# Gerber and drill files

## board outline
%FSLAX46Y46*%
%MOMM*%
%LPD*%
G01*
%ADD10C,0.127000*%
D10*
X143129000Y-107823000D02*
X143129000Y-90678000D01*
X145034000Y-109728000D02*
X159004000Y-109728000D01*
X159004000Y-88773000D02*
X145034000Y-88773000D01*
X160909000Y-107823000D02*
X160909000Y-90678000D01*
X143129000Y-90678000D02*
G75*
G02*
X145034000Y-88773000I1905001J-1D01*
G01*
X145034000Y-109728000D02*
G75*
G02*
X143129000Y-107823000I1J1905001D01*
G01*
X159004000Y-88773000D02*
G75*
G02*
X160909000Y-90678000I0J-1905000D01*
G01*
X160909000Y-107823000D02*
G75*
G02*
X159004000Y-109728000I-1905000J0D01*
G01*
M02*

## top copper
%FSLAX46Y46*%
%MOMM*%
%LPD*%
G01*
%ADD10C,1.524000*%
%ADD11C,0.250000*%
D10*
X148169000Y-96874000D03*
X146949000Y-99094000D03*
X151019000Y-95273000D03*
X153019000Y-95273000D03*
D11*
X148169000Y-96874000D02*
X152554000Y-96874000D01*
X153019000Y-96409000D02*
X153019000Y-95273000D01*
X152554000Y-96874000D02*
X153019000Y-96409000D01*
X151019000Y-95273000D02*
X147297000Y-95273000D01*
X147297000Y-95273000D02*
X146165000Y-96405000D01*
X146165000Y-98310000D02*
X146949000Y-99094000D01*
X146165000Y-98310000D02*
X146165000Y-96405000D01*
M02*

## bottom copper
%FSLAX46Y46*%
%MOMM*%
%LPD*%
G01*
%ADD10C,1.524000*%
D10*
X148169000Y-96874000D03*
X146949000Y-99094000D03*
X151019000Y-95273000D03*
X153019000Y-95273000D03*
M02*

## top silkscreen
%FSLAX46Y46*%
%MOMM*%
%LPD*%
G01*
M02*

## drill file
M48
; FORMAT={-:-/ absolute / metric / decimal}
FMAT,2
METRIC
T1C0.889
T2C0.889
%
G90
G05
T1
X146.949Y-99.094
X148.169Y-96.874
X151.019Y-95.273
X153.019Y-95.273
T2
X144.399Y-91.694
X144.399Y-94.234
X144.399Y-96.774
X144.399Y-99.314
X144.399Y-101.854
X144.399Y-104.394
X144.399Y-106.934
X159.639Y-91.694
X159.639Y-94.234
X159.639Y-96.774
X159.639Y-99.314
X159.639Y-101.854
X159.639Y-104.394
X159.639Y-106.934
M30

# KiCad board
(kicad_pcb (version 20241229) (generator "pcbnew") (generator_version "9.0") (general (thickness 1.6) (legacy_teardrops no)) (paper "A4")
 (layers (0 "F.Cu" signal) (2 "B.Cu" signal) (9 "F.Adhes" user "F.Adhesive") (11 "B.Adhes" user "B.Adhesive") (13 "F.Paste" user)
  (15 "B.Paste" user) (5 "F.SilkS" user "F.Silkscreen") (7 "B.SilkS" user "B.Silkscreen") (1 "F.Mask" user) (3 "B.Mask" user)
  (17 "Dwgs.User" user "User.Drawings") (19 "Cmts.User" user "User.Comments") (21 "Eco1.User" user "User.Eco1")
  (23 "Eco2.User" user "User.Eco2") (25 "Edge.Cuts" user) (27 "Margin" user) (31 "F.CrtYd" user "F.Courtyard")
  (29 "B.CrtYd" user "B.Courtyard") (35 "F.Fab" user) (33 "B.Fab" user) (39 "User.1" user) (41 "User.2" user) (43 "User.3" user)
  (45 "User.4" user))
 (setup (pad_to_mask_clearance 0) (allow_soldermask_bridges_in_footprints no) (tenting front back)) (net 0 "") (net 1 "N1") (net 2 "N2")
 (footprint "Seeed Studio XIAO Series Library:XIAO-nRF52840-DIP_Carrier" (layer "F.Cu") (at 152.019 99.314)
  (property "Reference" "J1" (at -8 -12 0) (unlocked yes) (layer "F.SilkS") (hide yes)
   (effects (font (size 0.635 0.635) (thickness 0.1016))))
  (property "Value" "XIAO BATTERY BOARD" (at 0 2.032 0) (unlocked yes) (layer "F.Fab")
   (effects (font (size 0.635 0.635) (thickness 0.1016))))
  (fp_line (start -8.89 8.509) (end -8.89 -8.636) (stroke (width 0.127) (type solid)) (layer "Edge.Cuts"))
  (fp_line (start -6.985 10.414) (end 6.985 10.414) (stroke (width 0.127) (type solid)) (layer "Edge.Cuts"))
  (fp_line (start 6.985 -10.541) (end -6.985 -10.541) (stroke (width 0.127) (type solid)) (layer "Edge.Cuts"))
  (fp_line (start 8.89 8.509) (end 8.89 -8.636) (stroke (width 0.127) (type solid)) (layer "Edge.Cuts"))
  (fp_arc (start -8.89 -8.636) (mid -8.332038 -9.983038) (end -6.985 -10.541) (stroke (width 0.127) (type solid)) (layer "Edge.Cuts"))
  (fp_arc (start -6.985 10.414) (mid -8.332038 9.856038) (end -8.89 8.509) (stroke (width 0.127) (type solid)) (layer "Edge.Cuts"))
  (fp_arc (start 6.985 -10.541) (mid 8.332038 -9.983038) (end 8.89 -8.636) (stroke (width 0.127) (type solid)) (layer "Edge.Cuts"))
  (fp_arc (start 8.89 8.509) (mid 8.332038 9.856038) (end 6.985 10.414) (stroke (width 0.127) (type solid)) (layer "Edge.Cuts"))
  (pad "" np_thru_hole circle (at -7.62 -7.62 180) (size 1.524 1.524) (drill 0.889) (layers))
  (pad "" np_thru_hole circle (at -7.62 -5.08 180) (size 0.889 0.889) (drill 0.889) (layers))
  (pad "" np_thru_hole circle (at -7.62 -2.54 180) (size 1.524 1.524) (drill 0.889) (layers))
  (pad "" np_thru_hole circle (at -7.62 0 180) (size 1.524 1.524) (drill 0.889) (layers))
  (pad "" np_thru_hole circle (at -7.62 2.54 180) (size 1.524 1.524) (drill 0.889) (layers))
  (pad "" np_thru_hole circle (at -7.62 5.08 180) (size 1.524 1.524) (drill 0.889) (layers))
  (pad "" np_thru_hole circle (at -7.62 7.62 180) (size 1.524 1.524) (drill 0.889) (layers))
  (pad "" np_thru_hole circle (at 7.62 -7.62) (size 1.524 1.524) (drill 0.889) (layers))
  (pad "" np_thru_hole circle (at 7.62 -5.08) (size 1.524 1.524) (drill 0.889) (layers))
  (pad "" np_thru_hole circle (at 7.62 -2.54) (size 1.524 1.524) (drill 0.889) (layers))
  (pad "" np_thru_hole circle (at 7.62 0) (size 1.524 1.524) (drill 0.889) (layers))
  (pad "" np_thru_hole circle (at 7.62 2.54) (size 1.524 1.524) (drill 0.889) (layers))
  (pad "" np_thru_hole circle (at 7.62 5.08) (size 1.524 1.524) (drill 0.889) (layers))
  (pad "" np_thru_hole circle (at 7.62 7.62) (size 1.524 1.524) (drill 0.889) (layers))
  (pad "1" thru_hole circle (at -3.85 -2.44) (size 1.524 1.524) (drill 0.889) (layers "*.Cu" "*.Mask") (remove_unused_layers no)
   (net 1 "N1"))
  (pad "2" thru_hole circle (at -5.07 -0.22) (size 1.524 1.524) (drill 0.889) (layers "*.Cu" "*.Mask") (remove_unused_layers no)
   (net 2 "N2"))
  (pad "3" thru_hole circle (at -1 -4.041) (size 1.524 1.524) (drill 0.889) (layers "*.Cu" "*.Mask") (remove_unused_layers no) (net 2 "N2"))
  (pad "4" thru_hole circle (at 1 -4.041) (size 1.524 1.524) (drill 0.889) (layers "*.Cu" "*.Mask") (remove_unused_layers no) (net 1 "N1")))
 (segment (start 148.169 96.874) (end 152.554 96.874) (width 0.25) (layer "F.Cu") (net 1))
 (segment (start 153.019 96.409) (end 153.019 95.273) (width 0.25) (layer "F.Cu") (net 1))
 (segment (start 152.554 96.874) (end 153.019 96.409) (width 0.25) (layer "F.Cu") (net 1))
 (segment (start 151.019 95.273) (end 147.297 95.273) (width 0.25) (layer "F.Cu") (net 2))
 (segment (start 147.297 95.273) (end 146.165 96.405) (width 0.25) (layer "F.Cu") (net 2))
 (segment (start 146.165 98.31) (end 146.949 99.094) (width 0.25) (layer "F.Cu") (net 2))
 (segment (start 146.165 98.31) (end 146.165 96.405) (width 0.25) (layer "F.Cu") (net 2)))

